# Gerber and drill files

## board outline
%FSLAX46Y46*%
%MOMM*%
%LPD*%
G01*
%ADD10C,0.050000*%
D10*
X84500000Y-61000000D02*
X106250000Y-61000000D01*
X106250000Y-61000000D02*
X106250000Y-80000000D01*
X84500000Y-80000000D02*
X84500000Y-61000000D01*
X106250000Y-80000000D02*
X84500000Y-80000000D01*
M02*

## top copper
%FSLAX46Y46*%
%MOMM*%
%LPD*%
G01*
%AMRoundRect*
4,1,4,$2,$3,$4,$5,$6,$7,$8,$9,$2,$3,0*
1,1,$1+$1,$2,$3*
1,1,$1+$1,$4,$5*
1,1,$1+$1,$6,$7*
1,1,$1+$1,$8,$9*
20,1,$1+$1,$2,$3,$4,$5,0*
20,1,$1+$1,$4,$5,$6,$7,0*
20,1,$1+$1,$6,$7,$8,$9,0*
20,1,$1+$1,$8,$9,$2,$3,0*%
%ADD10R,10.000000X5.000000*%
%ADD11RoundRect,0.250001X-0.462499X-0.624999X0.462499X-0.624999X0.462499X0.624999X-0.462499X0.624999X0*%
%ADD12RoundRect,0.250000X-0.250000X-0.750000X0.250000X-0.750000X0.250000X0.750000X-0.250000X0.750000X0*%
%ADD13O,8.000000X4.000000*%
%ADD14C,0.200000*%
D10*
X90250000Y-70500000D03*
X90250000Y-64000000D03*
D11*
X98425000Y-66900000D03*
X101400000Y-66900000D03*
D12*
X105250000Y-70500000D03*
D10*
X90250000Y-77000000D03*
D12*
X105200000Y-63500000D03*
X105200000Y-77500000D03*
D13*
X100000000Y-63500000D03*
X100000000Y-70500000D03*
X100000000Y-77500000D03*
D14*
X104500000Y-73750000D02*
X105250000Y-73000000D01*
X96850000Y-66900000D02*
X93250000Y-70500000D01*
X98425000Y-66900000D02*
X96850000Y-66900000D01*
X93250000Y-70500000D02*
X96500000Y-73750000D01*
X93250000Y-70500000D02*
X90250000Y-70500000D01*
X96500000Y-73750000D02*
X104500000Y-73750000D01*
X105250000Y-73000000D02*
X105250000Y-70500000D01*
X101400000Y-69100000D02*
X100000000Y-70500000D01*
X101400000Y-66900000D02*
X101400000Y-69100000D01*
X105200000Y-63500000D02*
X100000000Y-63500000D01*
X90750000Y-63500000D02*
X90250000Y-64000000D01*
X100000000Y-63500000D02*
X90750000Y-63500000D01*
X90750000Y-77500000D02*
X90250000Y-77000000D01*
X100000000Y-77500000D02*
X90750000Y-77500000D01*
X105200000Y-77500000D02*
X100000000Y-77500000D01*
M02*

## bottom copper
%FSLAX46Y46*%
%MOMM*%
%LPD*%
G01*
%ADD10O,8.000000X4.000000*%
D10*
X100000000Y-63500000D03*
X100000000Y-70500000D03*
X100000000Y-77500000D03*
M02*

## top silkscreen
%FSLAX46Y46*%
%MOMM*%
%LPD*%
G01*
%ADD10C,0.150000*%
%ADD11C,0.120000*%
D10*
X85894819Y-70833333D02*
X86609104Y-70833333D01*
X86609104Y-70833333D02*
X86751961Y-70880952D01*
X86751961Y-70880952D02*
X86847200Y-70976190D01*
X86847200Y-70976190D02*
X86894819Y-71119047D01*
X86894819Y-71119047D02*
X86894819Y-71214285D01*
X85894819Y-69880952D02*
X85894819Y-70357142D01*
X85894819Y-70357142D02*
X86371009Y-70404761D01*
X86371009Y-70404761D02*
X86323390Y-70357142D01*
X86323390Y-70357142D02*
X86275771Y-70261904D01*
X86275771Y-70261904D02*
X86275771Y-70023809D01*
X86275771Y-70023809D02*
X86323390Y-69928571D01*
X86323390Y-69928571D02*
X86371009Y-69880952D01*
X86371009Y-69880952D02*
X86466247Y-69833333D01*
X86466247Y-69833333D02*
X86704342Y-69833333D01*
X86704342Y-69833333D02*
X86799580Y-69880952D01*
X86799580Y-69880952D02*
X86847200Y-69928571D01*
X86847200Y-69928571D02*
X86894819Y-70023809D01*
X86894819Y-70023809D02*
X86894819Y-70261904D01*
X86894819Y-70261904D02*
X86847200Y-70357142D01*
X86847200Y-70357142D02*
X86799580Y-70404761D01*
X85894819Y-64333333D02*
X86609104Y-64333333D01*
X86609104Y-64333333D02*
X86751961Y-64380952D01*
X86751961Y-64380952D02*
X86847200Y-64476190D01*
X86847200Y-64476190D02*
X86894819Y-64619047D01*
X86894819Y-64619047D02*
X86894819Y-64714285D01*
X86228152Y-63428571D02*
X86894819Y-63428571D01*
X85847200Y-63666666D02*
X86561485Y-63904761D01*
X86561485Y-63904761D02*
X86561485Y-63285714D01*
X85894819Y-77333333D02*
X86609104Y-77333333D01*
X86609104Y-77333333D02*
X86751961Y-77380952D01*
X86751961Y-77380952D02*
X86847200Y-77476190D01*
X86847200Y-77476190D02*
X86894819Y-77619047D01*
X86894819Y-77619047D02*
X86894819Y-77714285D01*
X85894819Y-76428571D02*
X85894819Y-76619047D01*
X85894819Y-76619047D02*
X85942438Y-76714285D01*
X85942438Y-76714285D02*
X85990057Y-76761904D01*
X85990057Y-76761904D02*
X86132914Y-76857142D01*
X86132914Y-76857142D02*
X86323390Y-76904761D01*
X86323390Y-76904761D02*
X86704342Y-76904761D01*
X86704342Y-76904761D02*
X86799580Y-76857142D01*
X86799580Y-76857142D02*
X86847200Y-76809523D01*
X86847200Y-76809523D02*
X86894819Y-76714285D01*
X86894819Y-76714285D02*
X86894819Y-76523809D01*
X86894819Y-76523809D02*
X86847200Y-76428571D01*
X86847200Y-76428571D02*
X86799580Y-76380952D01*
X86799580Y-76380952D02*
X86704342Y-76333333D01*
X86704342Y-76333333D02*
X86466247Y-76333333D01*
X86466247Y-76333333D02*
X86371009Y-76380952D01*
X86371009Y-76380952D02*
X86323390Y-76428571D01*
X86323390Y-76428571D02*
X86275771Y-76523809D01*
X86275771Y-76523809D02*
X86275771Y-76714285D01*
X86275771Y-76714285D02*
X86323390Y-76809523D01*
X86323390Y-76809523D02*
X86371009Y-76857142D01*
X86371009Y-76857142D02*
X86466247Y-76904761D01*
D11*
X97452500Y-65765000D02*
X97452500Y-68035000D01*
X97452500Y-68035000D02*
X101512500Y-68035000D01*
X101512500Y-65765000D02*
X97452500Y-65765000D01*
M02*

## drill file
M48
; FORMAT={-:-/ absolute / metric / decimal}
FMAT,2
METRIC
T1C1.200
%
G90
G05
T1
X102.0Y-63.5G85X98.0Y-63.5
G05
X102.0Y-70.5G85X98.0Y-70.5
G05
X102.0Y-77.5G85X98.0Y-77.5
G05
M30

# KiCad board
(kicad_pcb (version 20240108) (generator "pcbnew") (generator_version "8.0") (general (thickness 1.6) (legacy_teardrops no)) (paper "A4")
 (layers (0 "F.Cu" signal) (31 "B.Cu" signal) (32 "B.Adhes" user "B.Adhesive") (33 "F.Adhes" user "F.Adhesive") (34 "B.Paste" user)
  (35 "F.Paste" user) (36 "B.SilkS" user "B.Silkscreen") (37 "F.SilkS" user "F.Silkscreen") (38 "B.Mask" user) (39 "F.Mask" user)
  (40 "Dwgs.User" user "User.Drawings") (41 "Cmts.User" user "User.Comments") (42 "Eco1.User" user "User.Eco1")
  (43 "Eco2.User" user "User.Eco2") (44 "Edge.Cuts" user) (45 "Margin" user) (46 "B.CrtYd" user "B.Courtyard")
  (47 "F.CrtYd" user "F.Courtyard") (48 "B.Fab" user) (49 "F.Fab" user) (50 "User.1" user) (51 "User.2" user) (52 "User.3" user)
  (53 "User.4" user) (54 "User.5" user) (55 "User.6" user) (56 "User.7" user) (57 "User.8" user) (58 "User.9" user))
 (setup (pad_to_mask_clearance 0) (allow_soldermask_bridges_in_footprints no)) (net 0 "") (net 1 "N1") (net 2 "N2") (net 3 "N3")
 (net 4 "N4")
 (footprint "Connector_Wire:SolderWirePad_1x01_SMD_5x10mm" (layer "F.Cu") (at 90.25 70.5 90)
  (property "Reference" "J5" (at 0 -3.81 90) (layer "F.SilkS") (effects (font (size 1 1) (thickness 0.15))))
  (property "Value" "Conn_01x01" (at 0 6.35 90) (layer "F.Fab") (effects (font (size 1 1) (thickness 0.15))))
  (pad "1" smd rect (at 0 0 90) (size 5 10) (layers "F.Cu" "F.Paste" "F.Mask") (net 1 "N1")))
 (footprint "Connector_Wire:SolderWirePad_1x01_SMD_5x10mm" (layer "F.Cu") (at 90.25 64 90)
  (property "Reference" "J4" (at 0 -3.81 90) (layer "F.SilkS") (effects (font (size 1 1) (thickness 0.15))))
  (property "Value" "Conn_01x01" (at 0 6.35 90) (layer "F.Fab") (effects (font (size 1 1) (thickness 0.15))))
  (pad "1" smd rect (at 0 0 90) (size 5 10) (layers "F.Cu" "F.Paste" "F.Mask") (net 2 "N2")))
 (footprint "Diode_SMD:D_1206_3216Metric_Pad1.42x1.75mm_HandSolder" (layer "F.Cu") (at 99.9125 66.9)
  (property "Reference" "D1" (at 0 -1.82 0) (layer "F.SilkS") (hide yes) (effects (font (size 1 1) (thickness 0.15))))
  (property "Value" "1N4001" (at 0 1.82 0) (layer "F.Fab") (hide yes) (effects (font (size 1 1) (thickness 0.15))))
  (fp_line (start -2.46 -1.135) (end -2.46 1.135) (stroke (width 0.12) (type solid)) (layer "F.SilkS"))
  (fp_line (start -2.46 1.135) (end 1.6 1.135) (stroke (width 0.12) (type solid)) (layer "F.SilkS"))
  (fp_line (start 1.6 -1.135) (end -2.46 -1.135) (stroke (width 0.12) (type solid)) (layer "F.SilkS"))
  (pad "1" smd roundrect (at -1.4875 0) (size 1.425 1.75) (layers "F.Cu" "F.Paste" "F.Mask") (roundrect_rratio 0.175439) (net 1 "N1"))
  (pad "2" smd roundrect (at 1.4875 0) (size 1.425 1.75) (layers "F.Cu" "F.Paste" "F.Mask") (roundrect_rratio 0.175439) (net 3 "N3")))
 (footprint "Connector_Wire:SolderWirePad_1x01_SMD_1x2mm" (layer "F.Cu") (at 105.25 70.5)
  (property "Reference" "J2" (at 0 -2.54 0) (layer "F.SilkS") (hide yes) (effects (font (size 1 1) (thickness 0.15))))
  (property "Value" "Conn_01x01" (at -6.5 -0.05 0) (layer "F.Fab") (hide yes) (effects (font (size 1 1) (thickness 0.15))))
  (pad "1" smd roundrect (at 0 0) (size 1 2) (layers "F.Cu" "F.Paste" "F.Mask") (roundrect_rratio 0.25) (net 1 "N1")))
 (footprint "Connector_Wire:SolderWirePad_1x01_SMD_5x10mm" (layer "F.Cu") (at 90.25 77 90)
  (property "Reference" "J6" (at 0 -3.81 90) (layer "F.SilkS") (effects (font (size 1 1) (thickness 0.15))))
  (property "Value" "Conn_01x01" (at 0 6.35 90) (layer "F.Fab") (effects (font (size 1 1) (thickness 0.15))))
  (pad "1" smd rect (at 0 0 90) (size 5 10) (layers "F.Cu" "F.Paste" "F.Mask") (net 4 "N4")))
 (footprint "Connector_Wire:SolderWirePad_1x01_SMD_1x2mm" (layer "F.Cu") (at 105.2 63.5)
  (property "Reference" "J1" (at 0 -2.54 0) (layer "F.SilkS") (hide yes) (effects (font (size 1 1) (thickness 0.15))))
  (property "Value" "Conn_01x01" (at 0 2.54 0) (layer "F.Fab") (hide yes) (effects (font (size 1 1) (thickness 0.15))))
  (pad "1" smd roundrect (at 0 0) (size 1 2) (layers "F.Cu" "F.Paste" "F.Mask") (roundrect_rratio 0.25) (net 2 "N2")))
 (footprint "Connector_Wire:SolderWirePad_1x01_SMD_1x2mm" (layer "F.Cu") (at 105.2 77.5)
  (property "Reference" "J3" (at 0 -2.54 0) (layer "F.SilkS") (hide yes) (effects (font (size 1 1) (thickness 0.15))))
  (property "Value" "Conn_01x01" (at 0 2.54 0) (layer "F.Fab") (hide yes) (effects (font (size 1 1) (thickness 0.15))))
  (pad "1" smd roundrect (at 0 0) (size 1 2) (layers "F.Cu" "F.Paste" "F.Mask") (roundrect_rratio 0.25) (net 4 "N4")))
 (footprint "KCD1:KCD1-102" (layer "B.Cu") (at 100 70.5 180)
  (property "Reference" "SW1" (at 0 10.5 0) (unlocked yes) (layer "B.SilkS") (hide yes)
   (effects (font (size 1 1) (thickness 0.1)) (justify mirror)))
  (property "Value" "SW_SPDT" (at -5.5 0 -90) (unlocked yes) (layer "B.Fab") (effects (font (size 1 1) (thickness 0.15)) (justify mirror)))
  (pad "1" thru_hole oval (at 0 7 180) (size 8 4) (drill oval 5.2 1.2) (layers "*.Cu" "*.Mask") (remove_unused_layers no) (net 2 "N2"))
  (pad "2" thru_hole oval (at 0 0 180) (size 8 4) (drill oval 5.2 1.2) (layers "*.Cu" "*.Mask") (remove_unused_layers no) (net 3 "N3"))
  (pad "3" thru_hole oval (at 0 -7 180) (size 8 4) (drill oval 5.2 1.2) (layers "*.Cu" "*.Mask") (remove_unused_layers no) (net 4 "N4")))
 (gr_line (start 84.5 61) (end 106.25 61) (stroke (width 0.05) (type default)) (layer "Edge.Cuts"))
 (gr_line (start 106.25 61) (end 106.25 80) (stroke (width 0.05) (type default)) (layer "Edge.Cuts"))
 (gr_line (start 84.5 80) (end 84.5 61) (stroke (width 0.05) (type default)) (layer "Edge.Cuts"))
 (gr_line (start 106.25 80) (end 84.5 80) (stroke (width 0.05) (type default)) (layer "Edge.Cuts"))
 (segment (start 104.5 73.75) (end 105.25 73) (width 0.2) (layer "F.Cu") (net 1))
 (segment (start 96.85 66.9) (end 93.25 70.5) (width 0.2) (layer "F.Cu") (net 1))
 (segment (start 98.425 66.9) (end 96.85 66.9) (width 0.2) (layer "F.Cu") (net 1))
 (segment (start 93.25 70.5) (end 96.5 73.75) (width 0.2) (layer "F.Cu") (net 1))
 (segment (start 93.25 70.5) (end 90.25 70.5) (width 0.2) (layer "F.Cu") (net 1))
 (segment (start 96.5 73.75) (end 104.5 73.75) (width 0.2) (layer "F.Cu") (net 1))
 (segment (start 105.25 73) (end 105.25 70.5) (width 0.2) (layer "F.Cu") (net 1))
 (segment (start 101.4 69.1) (end 100 70.5) (width 0.2) (layer "F.Cu") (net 3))
 (segment (start 101.4 66.9) (end 101.4 69.1) (width 0.2) (layer "F.Cu") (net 3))
 (segment (start 105.2 63.5) (end 100 63.5) (width 0.2) (layer "F.Cu") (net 2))
 (segment (start 90.75 63.5) (end 90.25 64) (width 0.2) (layer "F.Cu") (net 2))
 (segment (start 100 63.5) (end 90.75 63.5) (width 0.2) (layer "F.Cu") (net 2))
 (segment (start 90.75 77.5) (end 90.25 77) (width 0.2) (layer "F.Cu") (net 4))
 (segment (start 100 77.5) (end 90.75 77.5) (width 0.2) (layer "F.Cu") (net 4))
 (segment (start 105.2 77.5) (end 100 77.5) (width 0.2) (layer "F.Cu") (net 4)))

